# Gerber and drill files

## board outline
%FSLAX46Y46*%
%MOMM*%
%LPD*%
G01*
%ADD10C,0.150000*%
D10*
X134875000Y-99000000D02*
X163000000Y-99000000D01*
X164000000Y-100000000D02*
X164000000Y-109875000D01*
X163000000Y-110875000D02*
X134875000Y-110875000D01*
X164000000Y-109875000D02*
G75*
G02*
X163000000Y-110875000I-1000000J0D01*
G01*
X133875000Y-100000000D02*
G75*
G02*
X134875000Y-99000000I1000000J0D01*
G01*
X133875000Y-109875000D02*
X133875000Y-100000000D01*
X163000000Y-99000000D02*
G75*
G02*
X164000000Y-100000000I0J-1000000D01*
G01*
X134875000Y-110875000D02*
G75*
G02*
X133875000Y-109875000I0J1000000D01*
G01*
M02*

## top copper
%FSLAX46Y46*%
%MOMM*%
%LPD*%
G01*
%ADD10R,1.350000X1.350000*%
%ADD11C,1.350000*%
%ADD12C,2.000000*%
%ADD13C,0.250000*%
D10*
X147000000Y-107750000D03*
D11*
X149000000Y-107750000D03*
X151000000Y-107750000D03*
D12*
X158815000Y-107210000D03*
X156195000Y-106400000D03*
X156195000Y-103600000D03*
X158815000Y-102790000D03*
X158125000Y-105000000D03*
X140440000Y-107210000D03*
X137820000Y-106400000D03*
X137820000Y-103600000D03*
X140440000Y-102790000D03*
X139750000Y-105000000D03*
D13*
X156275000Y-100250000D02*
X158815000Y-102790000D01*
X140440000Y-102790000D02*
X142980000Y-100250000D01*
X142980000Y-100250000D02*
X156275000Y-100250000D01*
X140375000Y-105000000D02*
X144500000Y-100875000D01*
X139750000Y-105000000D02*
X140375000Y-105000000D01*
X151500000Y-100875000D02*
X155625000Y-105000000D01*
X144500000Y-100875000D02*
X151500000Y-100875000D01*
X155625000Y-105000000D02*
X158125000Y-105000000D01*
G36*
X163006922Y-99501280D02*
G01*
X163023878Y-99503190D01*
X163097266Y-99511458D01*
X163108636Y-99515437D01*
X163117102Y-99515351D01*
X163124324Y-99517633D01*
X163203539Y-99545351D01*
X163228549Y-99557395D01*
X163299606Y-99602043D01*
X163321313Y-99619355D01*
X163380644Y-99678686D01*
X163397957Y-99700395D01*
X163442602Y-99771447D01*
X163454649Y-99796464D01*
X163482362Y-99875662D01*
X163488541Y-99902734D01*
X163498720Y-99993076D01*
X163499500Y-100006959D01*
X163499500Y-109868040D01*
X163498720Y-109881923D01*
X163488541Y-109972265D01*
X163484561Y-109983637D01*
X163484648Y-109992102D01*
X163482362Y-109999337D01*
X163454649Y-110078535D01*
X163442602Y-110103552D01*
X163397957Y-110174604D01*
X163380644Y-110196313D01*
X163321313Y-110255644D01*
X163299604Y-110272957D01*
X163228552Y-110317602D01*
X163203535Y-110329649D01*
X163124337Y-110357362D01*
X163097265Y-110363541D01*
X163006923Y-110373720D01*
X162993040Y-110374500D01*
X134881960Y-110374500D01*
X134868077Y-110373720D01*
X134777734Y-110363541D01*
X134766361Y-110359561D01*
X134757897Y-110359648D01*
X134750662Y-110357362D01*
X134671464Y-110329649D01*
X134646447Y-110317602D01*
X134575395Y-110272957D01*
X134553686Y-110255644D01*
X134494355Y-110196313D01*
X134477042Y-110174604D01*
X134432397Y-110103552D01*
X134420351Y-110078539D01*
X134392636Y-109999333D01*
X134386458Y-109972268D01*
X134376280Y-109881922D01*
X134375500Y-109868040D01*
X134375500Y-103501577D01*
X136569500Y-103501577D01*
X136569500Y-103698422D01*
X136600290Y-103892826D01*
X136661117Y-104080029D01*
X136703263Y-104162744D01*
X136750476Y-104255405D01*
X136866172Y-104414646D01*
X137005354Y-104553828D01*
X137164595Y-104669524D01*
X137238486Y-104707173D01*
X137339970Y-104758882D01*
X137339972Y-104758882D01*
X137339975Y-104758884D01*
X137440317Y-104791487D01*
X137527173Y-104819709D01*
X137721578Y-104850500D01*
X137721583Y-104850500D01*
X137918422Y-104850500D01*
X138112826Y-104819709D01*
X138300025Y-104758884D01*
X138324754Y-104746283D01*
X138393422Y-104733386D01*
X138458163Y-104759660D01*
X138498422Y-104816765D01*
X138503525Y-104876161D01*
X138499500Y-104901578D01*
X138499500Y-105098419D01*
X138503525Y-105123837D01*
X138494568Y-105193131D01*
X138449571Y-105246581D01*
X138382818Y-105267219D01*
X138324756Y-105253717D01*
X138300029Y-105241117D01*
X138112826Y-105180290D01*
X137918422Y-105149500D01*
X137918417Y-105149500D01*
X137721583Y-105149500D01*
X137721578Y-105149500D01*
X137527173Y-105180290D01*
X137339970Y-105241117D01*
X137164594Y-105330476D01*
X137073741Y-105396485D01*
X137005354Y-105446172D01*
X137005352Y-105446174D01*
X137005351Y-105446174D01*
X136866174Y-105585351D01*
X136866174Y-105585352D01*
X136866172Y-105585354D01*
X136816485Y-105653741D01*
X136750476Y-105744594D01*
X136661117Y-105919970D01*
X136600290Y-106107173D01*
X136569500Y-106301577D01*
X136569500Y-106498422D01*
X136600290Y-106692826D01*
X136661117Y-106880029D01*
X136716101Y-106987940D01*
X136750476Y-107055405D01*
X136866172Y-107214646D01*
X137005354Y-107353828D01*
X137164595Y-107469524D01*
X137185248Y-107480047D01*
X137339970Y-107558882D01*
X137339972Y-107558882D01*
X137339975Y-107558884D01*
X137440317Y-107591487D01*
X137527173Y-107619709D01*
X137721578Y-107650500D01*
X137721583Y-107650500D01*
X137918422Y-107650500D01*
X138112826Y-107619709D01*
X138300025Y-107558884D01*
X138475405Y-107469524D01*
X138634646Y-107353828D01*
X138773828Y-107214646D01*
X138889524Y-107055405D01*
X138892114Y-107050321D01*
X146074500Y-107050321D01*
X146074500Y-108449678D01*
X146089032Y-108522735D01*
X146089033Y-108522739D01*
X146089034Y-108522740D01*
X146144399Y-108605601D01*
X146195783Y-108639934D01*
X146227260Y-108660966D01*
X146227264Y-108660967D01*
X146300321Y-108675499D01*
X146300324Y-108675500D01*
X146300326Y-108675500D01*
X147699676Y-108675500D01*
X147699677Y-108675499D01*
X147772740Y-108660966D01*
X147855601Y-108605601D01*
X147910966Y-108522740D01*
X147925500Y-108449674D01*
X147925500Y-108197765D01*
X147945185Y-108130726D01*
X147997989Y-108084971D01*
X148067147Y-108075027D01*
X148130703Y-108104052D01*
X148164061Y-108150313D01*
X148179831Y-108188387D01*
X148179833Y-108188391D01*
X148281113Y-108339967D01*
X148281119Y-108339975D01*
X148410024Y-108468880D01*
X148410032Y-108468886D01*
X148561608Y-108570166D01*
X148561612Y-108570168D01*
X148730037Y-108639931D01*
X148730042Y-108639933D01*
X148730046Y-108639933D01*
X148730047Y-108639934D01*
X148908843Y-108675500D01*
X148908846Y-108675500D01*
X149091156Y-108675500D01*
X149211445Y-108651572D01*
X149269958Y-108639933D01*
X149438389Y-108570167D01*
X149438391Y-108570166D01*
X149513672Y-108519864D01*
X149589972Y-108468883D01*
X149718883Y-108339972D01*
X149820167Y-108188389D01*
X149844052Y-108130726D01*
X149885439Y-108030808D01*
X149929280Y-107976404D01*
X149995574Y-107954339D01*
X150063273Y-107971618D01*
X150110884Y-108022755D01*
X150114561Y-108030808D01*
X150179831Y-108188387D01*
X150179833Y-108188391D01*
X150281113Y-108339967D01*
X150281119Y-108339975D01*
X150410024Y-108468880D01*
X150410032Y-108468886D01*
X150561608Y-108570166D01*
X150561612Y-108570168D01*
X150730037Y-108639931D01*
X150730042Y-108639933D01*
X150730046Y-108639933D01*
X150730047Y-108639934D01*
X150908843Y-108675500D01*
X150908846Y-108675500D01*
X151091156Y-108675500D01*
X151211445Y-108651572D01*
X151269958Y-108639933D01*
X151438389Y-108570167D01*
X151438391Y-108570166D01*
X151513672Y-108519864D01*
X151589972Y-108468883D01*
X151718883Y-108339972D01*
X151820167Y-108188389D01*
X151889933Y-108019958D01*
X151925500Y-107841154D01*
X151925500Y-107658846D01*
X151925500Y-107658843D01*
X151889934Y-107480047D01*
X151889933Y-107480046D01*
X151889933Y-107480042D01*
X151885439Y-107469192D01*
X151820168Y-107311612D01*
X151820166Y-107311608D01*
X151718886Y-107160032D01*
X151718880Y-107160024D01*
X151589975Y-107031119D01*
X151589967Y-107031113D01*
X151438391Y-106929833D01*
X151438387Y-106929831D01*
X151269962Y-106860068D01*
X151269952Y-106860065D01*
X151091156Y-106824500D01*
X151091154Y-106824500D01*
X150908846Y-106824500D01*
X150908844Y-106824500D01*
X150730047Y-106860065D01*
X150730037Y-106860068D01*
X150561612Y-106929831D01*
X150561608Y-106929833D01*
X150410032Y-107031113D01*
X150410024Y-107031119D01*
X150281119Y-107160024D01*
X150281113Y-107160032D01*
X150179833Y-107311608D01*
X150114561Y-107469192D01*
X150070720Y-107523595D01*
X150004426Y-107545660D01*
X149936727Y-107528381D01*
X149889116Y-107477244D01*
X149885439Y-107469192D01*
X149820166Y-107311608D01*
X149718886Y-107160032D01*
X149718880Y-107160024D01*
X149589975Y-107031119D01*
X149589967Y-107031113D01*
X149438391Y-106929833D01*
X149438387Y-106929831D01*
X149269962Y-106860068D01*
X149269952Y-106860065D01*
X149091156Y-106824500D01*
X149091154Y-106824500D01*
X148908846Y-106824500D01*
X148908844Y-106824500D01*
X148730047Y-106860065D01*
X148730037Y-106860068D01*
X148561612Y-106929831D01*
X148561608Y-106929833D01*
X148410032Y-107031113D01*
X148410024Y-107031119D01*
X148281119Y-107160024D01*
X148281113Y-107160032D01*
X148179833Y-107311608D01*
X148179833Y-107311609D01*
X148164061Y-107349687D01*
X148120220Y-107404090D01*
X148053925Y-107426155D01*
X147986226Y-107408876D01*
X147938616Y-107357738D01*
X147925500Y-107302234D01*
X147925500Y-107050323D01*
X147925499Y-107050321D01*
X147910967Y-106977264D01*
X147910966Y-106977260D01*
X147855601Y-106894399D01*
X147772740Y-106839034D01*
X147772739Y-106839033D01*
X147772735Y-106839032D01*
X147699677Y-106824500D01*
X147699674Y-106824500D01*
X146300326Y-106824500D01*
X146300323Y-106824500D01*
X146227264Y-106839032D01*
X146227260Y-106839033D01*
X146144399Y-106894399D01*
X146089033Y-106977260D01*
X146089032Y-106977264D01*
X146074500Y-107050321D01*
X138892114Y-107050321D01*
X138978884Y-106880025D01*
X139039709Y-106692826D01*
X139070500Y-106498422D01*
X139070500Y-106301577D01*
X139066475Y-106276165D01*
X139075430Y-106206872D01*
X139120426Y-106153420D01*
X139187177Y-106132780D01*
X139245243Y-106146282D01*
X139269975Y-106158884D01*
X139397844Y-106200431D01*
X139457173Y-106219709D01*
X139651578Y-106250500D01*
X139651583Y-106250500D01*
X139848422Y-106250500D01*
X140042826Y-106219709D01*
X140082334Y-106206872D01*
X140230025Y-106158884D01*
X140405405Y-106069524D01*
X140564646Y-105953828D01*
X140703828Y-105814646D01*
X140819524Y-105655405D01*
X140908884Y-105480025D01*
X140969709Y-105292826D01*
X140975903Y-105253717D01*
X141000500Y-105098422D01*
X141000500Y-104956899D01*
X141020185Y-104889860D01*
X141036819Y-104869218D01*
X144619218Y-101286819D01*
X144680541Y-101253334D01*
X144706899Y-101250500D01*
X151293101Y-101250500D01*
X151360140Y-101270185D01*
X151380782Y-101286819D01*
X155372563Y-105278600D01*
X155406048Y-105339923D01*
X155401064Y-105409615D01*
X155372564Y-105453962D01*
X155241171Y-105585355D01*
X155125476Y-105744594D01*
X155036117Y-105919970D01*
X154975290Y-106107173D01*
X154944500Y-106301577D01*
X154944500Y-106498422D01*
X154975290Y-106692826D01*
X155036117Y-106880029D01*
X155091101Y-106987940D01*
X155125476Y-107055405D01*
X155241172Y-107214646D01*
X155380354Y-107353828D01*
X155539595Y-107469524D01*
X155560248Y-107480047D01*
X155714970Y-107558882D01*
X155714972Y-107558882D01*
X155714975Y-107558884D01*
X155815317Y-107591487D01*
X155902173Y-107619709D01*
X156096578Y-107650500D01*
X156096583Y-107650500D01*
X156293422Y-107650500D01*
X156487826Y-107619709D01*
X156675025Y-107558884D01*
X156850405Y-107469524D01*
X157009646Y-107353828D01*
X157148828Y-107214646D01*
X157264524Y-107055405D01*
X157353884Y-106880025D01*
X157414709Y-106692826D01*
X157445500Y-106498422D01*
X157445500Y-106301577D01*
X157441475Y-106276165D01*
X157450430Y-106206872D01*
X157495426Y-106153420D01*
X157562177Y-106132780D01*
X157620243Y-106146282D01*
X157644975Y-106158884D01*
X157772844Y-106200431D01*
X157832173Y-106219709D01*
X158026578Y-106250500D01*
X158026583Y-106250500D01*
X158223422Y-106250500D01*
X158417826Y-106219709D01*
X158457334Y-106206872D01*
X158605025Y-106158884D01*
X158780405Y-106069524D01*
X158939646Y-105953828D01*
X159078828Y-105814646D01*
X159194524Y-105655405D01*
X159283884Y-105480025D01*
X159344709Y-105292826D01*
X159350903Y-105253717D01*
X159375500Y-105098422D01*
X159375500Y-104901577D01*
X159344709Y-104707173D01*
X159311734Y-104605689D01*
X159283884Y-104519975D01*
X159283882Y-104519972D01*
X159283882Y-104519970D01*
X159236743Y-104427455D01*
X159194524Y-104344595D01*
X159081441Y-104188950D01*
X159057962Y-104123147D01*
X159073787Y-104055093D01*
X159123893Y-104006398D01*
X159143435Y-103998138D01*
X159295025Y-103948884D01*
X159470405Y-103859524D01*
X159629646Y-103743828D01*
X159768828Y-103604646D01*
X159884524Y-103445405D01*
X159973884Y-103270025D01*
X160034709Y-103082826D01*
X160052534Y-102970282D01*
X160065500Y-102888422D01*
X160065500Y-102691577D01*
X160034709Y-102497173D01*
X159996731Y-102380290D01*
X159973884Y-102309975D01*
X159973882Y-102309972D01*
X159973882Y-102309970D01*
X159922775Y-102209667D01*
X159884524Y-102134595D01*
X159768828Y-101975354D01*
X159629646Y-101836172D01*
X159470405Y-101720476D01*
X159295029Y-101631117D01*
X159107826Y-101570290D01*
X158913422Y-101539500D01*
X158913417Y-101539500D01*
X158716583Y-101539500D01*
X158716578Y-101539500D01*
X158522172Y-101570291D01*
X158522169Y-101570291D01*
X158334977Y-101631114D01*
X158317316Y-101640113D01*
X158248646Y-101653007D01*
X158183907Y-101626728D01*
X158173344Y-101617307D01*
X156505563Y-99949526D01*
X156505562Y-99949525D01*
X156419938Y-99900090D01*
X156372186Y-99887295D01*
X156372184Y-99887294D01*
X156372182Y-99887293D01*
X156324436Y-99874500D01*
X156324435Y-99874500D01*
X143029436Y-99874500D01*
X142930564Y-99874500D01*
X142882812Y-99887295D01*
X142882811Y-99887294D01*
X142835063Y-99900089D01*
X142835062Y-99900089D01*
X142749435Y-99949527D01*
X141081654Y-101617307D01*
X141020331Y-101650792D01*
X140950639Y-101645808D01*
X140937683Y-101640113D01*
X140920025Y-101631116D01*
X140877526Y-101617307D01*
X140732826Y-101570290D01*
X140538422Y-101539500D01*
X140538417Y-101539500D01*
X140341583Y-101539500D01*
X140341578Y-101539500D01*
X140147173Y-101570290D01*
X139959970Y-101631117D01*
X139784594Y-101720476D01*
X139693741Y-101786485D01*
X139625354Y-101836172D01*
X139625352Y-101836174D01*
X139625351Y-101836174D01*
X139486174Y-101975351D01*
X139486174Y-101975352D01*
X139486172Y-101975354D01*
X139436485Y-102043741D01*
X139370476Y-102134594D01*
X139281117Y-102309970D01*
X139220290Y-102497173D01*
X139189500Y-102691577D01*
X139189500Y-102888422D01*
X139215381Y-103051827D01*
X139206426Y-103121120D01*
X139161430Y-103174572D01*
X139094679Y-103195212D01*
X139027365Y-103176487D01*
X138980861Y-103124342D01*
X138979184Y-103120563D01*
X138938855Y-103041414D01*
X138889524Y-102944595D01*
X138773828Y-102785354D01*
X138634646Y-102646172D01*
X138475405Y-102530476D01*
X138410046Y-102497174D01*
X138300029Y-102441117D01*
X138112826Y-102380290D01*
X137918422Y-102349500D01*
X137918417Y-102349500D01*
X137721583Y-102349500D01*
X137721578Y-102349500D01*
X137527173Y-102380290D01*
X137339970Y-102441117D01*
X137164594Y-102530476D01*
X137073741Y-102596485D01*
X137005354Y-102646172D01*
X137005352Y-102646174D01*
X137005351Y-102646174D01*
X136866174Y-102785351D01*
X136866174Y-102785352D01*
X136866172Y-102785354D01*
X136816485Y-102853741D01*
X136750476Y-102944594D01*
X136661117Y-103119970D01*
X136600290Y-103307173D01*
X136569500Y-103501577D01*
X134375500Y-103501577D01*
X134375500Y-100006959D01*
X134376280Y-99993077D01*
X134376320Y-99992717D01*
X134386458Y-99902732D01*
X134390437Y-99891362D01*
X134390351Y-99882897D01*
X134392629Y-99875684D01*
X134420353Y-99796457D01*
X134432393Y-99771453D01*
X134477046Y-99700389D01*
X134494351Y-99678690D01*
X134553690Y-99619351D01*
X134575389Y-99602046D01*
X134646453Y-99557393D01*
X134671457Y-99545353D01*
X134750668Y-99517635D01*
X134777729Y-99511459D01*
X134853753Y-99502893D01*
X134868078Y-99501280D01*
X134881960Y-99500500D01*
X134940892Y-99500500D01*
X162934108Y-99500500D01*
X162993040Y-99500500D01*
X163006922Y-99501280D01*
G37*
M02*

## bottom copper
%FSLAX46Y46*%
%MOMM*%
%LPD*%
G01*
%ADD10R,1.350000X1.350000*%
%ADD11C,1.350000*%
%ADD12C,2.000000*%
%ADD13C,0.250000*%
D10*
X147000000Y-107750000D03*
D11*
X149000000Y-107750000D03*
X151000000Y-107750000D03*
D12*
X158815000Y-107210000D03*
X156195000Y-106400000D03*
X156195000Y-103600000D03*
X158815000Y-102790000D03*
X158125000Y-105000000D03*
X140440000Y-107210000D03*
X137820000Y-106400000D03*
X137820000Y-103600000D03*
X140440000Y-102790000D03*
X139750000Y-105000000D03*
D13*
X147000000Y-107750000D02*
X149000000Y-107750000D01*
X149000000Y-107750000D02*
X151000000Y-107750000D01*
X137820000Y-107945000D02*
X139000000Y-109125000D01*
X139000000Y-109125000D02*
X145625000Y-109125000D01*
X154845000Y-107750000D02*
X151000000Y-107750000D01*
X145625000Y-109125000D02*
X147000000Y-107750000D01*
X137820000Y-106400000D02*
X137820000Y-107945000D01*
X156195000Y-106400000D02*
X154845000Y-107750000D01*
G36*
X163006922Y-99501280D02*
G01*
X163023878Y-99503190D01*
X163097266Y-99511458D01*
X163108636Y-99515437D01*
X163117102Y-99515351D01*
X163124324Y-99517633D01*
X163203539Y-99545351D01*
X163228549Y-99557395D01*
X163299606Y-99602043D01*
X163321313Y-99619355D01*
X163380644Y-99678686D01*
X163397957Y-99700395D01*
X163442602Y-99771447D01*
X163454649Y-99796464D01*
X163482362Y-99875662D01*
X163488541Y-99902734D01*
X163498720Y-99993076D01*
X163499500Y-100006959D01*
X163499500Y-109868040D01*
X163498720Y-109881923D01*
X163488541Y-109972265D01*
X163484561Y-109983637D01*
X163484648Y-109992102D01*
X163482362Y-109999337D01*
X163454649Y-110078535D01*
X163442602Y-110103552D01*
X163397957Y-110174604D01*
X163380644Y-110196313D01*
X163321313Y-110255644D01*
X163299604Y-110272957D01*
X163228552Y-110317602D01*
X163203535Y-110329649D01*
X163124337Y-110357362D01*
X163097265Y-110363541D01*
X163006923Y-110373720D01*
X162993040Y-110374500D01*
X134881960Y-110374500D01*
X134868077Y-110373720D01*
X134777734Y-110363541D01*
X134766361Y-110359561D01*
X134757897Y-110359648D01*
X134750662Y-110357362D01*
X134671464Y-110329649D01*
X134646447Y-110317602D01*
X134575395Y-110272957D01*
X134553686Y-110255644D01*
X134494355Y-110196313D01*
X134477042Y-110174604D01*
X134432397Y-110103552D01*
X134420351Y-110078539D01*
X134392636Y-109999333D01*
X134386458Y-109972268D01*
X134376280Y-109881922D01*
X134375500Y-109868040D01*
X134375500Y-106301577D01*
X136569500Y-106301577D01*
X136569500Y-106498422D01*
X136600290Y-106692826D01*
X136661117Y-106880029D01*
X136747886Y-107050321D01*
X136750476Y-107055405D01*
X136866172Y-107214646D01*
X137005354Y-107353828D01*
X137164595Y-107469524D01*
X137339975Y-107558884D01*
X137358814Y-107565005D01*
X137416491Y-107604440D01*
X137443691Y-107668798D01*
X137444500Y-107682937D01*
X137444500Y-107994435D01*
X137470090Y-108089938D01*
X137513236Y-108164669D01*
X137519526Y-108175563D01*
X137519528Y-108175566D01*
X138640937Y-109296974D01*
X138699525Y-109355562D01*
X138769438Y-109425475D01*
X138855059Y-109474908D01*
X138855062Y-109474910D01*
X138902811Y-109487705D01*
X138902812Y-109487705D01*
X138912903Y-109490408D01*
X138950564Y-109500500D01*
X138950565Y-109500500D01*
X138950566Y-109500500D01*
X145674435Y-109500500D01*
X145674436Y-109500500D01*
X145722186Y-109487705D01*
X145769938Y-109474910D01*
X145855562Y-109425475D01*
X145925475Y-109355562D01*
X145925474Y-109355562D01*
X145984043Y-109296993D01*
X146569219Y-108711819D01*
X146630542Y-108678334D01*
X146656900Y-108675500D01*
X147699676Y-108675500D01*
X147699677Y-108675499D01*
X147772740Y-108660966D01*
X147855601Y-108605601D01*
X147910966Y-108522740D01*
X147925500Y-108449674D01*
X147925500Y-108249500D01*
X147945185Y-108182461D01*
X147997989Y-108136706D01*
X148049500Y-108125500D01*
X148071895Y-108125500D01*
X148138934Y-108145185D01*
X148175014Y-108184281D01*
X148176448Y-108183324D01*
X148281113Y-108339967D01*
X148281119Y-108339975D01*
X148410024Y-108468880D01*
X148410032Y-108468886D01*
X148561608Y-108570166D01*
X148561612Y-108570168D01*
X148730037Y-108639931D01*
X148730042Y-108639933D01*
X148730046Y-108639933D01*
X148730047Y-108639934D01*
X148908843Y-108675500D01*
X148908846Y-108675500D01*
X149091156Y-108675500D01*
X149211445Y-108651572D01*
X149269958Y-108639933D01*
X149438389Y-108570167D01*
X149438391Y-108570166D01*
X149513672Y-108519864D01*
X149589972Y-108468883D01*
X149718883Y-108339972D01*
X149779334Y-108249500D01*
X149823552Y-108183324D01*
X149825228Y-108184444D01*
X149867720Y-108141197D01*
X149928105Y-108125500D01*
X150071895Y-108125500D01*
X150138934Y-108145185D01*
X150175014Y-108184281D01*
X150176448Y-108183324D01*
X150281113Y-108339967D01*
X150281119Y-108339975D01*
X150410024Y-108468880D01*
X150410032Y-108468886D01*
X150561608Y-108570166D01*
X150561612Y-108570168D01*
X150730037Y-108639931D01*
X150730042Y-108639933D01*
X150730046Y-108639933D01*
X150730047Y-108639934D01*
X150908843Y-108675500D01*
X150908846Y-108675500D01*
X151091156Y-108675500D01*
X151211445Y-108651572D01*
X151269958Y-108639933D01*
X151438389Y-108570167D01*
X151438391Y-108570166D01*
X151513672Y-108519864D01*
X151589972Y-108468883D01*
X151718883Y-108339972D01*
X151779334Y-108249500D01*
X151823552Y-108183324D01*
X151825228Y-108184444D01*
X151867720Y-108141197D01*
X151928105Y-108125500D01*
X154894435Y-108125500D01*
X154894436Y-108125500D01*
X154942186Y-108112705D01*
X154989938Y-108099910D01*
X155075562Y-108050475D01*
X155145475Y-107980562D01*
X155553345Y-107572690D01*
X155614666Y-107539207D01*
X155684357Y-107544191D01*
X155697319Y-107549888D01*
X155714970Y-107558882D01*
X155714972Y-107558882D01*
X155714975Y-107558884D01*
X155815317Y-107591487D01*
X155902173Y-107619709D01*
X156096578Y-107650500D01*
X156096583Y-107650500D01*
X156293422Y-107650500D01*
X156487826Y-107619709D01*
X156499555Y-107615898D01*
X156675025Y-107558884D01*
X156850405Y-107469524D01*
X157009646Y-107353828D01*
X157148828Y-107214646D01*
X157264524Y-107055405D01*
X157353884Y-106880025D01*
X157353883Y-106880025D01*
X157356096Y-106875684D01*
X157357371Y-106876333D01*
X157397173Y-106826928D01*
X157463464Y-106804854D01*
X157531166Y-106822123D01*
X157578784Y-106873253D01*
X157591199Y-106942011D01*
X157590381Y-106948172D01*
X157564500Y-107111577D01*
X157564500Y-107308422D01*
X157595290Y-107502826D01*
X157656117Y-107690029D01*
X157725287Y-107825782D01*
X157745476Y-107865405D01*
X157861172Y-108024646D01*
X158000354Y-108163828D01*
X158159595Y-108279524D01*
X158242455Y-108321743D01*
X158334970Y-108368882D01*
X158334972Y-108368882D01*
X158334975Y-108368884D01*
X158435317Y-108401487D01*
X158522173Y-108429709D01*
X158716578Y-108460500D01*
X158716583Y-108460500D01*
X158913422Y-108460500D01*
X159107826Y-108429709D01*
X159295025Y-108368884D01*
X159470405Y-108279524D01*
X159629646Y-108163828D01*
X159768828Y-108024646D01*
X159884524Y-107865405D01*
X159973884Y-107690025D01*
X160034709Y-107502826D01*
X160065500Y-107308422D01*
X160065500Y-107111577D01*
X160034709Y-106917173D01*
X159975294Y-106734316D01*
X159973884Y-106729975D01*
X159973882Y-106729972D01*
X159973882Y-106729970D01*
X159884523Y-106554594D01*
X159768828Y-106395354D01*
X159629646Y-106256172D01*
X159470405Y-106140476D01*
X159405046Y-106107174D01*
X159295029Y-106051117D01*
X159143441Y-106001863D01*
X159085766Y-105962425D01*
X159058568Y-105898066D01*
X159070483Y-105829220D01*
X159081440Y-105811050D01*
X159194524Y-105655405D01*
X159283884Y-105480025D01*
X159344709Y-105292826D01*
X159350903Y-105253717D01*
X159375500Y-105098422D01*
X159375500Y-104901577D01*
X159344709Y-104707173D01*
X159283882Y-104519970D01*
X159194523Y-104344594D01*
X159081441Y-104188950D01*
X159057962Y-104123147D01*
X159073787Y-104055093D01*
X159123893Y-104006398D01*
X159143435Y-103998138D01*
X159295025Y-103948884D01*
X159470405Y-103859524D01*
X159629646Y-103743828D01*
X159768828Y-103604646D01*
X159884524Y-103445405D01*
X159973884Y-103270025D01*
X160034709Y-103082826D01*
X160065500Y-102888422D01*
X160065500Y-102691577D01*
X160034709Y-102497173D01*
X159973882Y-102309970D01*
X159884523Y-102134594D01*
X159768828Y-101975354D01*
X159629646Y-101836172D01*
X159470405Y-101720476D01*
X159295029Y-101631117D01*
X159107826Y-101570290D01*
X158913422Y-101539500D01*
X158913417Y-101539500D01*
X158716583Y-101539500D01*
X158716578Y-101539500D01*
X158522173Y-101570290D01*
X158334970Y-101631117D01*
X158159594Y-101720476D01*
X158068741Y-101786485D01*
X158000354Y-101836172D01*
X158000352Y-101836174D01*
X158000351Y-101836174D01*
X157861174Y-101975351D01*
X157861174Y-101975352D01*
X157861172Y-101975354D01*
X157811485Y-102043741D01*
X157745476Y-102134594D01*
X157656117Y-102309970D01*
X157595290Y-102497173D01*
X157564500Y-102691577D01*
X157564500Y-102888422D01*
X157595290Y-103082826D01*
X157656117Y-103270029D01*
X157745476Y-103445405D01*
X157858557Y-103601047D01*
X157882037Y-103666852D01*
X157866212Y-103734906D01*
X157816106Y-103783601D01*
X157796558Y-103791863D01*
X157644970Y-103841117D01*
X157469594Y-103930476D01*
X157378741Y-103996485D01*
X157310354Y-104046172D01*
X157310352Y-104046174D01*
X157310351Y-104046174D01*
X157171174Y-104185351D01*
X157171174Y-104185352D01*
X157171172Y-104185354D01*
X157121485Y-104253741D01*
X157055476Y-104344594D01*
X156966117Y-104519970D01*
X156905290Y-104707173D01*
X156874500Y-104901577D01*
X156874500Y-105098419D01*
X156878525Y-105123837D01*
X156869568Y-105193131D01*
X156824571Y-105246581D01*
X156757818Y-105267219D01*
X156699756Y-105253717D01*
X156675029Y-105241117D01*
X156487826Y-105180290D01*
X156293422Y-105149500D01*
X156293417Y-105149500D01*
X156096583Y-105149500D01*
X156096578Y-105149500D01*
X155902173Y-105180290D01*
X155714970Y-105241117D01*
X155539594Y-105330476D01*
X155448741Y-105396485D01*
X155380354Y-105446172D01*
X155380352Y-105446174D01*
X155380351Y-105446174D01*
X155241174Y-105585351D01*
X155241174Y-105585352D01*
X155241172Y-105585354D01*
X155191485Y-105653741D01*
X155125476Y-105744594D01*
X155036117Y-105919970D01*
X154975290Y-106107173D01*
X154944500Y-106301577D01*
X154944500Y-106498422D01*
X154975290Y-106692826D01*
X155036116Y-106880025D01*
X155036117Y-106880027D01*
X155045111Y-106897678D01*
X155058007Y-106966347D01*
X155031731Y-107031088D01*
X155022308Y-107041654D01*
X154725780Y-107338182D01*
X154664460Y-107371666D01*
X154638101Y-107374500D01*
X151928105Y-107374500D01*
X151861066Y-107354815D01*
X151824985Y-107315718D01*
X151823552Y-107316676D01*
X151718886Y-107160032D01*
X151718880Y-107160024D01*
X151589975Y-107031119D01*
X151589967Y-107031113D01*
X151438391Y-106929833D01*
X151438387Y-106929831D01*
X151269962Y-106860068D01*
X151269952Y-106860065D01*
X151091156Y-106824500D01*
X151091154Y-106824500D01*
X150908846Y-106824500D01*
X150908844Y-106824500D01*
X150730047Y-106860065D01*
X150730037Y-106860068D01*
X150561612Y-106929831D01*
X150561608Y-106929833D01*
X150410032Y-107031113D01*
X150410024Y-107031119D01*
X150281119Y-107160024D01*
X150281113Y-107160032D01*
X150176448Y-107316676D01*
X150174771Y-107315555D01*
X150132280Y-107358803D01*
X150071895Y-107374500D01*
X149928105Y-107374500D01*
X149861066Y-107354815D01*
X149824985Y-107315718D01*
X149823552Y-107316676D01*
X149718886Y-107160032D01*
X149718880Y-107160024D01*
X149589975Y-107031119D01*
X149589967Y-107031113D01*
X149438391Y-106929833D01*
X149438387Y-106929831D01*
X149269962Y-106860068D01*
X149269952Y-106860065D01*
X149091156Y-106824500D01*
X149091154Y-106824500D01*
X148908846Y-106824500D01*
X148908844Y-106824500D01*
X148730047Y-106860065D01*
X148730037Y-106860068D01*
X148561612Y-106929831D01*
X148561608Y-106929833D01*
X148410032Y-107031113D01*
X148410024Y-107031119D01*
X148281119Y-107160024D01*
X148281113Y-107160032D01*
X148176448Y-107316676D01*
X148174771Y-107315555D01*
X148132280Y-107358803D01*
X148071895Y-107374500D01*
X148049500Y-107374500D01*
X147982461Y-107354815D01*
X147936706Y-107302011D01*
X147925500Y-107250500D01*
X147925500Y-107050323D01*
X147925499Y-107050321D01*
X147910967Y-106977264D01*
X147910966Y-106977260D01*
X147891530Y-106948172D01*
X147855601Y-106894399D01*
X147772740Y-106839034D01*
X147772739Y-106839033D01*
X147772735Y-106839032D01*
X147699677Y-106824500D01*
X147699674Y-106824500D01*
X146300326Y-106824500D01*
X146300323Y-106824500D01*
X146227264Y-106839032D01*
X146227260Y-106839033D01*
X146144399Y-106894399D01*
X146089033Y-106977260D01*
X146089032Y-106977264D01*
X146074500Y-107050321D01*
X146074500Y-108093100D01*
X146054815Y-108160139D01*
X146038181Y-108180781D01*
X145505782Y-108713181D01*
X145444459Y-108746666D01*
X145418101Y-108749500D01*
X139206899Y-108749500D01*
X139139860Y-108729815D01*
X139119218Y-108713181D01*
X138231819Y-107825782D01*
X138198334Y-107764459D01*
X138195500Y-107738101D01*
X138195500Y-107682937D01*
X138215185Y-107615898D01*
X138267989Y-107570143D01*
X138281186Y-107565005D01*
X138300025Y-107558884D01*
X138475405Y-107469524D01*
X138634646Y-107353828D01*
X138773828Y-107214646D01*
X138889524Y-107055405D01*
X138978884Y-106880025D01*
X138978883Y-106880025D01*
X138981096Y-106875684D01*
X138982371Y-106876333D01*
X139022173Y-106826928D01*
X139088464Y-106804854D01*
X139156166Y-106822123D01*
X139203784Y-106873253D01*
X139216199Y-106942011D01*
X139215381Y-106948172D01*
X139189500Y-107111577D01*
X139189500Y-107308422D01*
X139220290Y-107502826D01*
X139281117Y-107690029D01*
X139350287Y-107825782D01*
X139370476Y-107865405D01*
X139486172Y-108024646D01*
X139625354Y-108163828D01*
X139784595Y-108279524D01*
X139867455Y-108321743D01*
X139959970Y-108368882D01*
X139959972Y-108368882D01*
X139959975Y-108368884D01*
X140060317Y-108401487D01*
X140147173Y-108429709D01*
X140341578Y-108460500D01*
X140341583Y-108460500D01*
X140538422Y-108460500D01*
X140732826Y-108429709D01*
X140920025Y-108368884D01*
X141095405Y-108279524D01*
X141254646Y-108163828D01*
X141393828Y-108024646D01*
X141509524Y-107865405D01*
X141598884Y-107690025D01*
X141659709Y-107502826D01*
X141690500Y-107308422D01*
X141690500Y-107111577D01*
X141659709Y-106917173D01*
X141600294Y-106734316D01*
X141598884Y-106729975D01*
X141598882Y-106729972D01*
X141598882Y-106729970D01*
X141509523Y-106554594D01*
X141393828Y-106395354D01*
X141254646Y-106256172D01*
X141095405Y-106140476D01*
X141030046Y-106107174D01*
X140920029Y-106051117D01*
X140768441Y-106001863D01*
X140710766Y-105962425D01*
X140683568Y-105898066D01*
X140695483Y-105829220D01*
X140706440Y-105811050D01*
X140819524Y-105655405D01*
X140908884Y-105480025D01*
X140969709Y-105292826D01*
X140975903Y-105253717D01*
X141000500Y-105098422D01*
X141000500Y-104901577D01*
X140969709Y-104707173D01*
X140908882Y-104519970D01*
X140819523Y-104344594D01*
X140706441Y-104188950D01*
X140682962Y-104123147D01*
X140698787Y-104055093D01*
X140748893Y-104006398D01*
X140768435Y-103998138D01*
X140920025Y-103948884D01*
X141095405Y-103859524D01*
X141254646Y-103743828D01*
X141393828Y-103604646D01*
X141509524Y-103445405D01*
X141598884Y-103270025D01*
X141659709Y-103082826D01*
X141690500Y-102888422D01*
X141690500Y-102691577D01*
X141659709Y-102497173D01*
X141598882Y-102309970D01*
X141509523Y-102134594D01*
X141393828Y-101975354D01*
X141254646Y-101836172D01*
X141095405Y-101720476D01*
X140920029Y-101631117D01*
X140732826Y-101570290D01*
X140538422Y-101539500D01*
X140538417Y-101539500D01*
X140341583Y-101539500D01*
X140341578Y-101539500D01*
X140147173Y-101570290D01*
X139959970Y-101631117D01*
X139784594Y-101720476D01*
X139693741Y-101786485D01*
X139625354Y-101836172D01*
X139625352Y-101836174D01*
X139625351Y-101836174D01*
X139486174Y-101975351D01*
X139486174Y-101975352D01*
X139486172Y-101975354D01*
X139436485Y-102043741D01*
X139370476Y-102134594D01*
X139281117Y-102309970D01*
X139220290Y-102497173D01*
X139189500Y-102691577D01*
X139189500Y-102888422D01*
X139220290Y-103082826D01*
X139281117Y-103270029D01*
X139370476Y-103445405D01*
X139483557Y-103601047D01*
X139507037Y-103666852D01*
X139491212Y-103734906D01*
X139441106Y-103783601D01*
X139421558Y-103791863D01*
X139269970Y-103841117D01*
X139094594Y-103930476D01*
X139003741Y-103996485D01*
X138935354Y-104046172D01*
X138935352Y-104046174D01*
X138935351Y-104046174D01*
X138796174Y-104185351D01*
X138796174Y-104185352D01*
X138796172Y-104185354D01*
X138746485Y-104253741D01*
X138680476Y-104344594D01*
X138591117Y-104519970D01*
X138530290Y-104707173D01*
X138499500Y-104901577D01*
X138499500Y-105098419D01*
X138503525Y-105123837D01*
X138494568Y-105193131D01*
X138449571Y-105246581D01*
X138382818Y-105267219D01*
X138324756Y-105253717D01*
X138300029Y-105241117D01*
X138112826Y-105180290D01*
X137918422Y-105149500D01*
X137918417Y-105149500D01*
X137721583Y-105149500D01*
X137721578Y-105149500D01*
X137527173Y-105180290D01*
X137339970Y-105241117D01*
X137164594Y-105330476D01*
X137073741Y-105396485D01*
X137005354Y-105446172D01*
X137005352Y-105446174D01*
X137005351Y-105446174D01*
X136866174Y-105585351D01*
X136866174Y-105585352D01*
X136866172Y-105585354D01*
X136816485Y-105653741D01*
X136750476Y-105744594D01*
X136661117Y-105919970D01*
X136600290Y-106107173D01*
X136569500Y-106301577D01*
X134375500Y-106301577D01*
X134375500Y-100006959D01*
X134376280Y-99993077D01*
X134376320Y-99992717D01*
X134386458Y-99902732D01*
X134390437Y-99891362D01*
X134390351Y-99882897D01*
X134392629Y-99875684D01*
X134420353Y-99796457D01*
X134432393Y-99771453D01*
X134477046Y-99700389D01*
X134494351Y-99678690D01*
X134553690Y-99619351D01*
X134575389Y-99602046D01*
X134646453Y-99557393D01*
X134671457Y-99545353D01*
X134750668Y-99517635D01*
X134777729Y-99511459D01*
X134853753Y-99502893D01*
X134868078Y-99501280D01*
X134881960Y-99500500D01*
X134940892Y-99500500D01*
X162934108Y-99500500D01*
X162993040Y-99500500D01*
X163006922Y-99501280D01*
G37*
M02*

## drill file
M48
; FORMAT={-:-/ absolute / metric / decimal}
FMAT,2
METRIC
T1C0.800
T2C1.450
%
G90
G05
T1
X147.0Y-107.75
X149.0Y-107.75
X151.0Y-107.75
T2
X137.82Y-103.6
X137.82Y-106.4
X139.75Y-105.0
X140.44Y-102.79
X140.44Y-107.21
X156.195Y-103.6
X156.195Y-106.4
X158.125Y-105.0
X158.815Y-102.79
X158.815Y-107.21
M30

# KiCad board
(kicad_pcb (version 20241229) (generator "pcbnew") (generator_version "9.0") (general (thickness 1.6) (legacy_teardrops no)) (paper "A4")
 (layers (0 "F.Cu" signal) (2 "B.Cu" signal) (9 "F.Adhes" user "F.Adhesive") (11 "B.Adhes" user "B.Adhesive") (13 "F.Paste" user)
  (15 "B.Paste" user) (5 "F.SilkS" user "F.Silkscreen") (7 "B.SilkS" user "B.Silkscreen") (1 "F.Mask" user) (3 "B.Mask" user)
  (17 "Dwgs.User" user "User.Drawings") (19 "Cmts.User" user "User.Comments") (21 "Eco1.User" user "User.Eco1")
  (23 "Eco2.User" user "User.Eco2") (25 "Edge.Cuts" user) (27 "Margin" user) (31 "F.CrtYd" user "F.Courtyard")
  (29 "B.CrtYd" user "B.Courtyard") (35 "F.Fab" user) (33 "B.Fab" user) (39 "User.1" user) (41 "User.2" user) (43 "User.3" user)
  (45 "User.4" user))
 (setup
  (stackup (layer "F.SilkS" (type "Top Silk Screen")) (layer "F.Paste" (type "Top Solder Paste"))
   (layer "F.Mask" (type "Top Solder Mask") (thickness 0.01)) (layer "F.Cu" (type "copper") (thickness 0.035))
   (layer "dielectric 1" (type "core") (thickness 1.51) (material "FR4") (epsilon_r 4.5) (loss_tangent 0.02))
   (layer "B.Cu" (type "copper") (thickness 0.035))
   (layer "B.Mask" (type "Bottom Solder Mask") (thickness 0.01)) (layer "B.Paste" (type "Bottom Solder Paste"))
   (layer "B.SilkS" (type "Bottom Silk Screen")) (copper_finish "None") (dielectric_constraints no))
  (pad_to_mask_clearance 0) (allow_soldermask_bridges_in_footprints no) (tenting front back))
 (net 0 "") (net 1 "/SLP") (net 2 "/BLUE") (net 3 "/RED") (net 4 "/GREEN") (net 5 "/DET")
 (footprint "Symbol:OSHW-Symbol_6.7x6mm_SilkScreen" (layer "F.Cu") (at 146 102.875)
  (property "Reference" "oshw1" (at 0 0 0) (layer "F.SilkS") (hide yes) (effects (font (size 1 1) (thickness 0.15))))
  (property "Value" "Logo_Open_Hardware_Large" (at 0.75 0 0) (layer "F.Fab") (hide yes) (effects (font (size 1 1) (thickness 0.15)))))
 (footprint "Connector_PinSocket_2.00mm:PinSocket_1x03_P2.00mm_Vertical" (layer "F.Cu") (at 147 107.75 90)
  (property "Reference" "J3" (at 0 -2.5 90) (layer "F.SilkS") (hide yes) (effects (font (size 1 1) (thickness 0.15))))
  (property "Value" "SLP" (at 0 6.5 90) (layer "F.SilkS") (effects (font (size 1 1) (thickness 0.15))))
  (pad "1" thru_hole rect (at 0 0 90) (size 1.35 1.35) (drill 0.8) (layers "*.Cu" "*.Mask") (remove_unused_layers no) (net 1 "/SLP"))
  (pad "2" thru_hole circle (at 0 2 90) (size 1.35 1.35) (drill 0.8) (layers "*.Cu" "*.Mask") (remove_unused_layers no) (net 1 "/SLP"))
  (pad "3" thru_hole circle (at 0 4 90) (size 1.35 1.35) (drill 0.8) (layers "*.Cu" "*.Mask") (remove_unused_layers no) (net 1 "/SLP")))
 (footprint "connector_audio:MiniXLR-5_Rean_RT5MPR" (layer "B.Cu") (at 158.125 105 90)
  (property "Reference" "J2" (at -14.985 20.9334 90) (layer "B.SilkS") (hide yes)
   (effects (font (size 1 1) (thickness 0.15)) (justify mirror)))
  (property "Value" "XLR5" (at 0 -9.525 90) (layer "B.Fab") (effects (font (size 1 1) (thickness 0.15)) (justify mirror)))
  (pad "1" thru_hole circle (at -2.21 0.69 270) (size 2 2) (drill 1.45) (layers "*.Cu" "*.Mask") (remove_unused_layers no) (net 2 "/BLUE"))
  (pad "2" thru_hole circle (at -1.4 -1.93 270) (size 2 2) (drill 1.45) (layers "*.Cu" "*.Mask") (remove_unused_layers no) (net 1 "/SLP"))
  (pad "3" thru_hole circle (at 1.4 -1.93 270) (size 2 2) (drill 1.45) (layers "*.Cu" "*.Mask") (remove_unused_layers no) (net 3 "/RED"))
  (pad "4" thru_hole circle (at 2.21 0.69 270) (size 2 2) (drill 1.45) (layers "*.Cu" "*.Mask") (remove_unused_layers no) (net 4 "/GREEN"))
  (pad "5" thru_hole circle (at 0 0 270) (size 2 2) (drill 1.45) (layers "*.Cu" "*.Mask") (remove_unused_layers no) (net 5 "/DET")))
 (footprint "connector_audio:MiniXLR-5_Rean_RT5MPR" (layer "B.Cu") (at 139.75 105 90)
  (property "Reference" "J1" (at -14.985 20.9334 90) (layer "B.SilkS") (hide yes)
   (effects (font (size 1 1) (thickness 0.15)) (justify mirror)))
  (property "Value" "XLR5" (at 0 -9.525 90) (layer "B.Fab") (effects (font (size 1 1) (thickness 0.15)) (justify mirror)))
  (pad "1" thru_hole circle (at -2.21 0.69 270) (size 2 2) (drill 1.45) (layers "*.Cu" "*.Mask") (remove_unused_layers no) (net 2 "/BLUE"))
  (pad "2" thru_hole circle (at -1.4 -1.93 270) (size 2 2) (drill 1.45) (layers "*.Cu" "*.Mask") (remove_unused_layers no) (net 1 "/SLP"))
  (pad "3" thru_hole circle (at 1.4 -1.93 270) (size 2 2) (drill 1.45) (layers "*.Cu" "*.Mask") (remove_unused_layers no) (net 3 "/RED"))
  (pad "4" thru_hole circle (at 2.21 0.69 270) (size 2 2) (drill 1.45) (layers "*.Cu" "*.Mask") (remove_unused_layers no) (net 4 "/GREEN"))
  (pad "5" thru_hole circle (at 0 0 270) (size 2 2) (drill 1.45) (layers "*.Cu" "*.Mask") (remove_unused_layers no) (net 5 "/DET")))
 (gr_line (start 134.875 99) (end 163 99) (stroke (width 0.15) (type default)) (layer "Edge.Cuts"))
 (gr_line (start 164 100) (end 164 109.875) (stroke (width 0.15) (type default)) (layer "Edge.Cuts"))
 (gr_line (start 163 110.875) (end 134.875 110.875) (stroke (width 0.15) (type default)) (layer "Edge.Cuts"))
 (gr_arc (start 164 109.875) (mid 163.707107 110.582107) (end 163 110.875) (stroke (width 0.15) (type default)) (layer "Edge.Cuts"))
 (gr_arc (start 133.875 100) (mid 134.167893 99.292893) (end 134.875 99) (stroke (width 0.15) (type default)) (layer "Edge.Cuts"))
 (gr_line (start 133.875 109.875) (end 133.875 100) (stroke (width 0.15) (type default)) (layer "Edge.Cuts"))
 (gr_arc (start 163 99) (mid 163.707107 99.292893) (end 164 100) (stroke (width 0.15) (type default)) (layer "Edge.Cuts"))
 (gr_arc (start 134.875 110.875) (mid 134.167893 110.582107) (end 133.875 109.875) (stroke (width 0.15) (type default)) (layer "Edge.Cuts"))
 (segment (start 156.275 100.25) (end 158.815 102.79) (width 0.25) (layer "F.Cu") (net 4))
 (segment (start 140.44 102.79) (end 142.98 100.25) (width 0.25) (layer "F.Cu") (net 4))
 (segment (start 142.98 100.25) (end 156.275 100.25) (width 0.25) (layer "F.Cu") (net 4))
 (segment (start 140.375 105) (end 144.5 100.875) (width 0.25) (layer "F.Cu") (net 5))
 (segment (start 139.75 105) (end 140.375 105) (width 0.25) (layer "F.Cu") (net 5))
 (segment (start 151.5 100.875) (end 155.625 105) (width 0.25) (layer "F.Cu") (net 5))
 (segment (start 144.5 100.875) (end 151.5 100.875) (width 0.25) (layer "F.Cu") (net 5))
 (segment (start 155.625 105) (end 158.125 105) (width 0.25) (layer "F.Cu") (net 5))
 (segment (start 147 107.75) (end 149 107.75) (width 0.25) (layer "B.Cu") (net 1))
 (segment (start 149 107.75) (end 151 107.75) (width 0.25) (layer "B.Cu") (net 1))
 (segment (start 137.82 107.945) (end 139 109.125) (width 0.25) (layer "B.Cu") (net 1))
 (segment (start 139 109.125) (end 145.625 109.125) (width 0.25) (layer "B.Cu") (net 1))
 (segment (start 154.845 107.75) (end 151 107.75) (width 0.25) (layer "B.Cu") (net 1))
 (segment (start 145.625 109.125) (end 147 107.75) (width 0.25) (layer "B.Cu") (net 1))
 (segment (start 137.82 106.4) (end 137.82 107.945) (width 0.25) (layer "B.Cu") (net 1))
 (segment (start 156.195 106.4) (end 154.845 107.75) (width 0.25) (layer "B.Cu") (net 1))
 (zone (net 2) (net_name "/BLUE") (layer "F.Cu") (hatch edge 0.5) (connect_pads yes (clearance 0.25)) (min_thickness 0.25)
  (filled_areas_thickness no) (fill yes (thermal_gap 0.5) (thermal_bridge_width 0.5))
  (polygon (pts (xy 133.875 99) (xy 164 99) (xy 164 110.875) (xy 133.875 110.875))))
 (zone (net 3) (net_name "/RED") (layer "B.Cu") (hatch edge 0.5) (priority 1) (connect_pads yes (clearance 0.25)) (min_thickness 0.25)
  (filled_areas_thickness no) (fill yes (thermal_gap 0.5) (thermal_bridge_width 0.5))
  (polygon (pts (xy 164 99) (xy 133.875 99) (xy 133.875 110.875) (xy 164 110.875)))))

